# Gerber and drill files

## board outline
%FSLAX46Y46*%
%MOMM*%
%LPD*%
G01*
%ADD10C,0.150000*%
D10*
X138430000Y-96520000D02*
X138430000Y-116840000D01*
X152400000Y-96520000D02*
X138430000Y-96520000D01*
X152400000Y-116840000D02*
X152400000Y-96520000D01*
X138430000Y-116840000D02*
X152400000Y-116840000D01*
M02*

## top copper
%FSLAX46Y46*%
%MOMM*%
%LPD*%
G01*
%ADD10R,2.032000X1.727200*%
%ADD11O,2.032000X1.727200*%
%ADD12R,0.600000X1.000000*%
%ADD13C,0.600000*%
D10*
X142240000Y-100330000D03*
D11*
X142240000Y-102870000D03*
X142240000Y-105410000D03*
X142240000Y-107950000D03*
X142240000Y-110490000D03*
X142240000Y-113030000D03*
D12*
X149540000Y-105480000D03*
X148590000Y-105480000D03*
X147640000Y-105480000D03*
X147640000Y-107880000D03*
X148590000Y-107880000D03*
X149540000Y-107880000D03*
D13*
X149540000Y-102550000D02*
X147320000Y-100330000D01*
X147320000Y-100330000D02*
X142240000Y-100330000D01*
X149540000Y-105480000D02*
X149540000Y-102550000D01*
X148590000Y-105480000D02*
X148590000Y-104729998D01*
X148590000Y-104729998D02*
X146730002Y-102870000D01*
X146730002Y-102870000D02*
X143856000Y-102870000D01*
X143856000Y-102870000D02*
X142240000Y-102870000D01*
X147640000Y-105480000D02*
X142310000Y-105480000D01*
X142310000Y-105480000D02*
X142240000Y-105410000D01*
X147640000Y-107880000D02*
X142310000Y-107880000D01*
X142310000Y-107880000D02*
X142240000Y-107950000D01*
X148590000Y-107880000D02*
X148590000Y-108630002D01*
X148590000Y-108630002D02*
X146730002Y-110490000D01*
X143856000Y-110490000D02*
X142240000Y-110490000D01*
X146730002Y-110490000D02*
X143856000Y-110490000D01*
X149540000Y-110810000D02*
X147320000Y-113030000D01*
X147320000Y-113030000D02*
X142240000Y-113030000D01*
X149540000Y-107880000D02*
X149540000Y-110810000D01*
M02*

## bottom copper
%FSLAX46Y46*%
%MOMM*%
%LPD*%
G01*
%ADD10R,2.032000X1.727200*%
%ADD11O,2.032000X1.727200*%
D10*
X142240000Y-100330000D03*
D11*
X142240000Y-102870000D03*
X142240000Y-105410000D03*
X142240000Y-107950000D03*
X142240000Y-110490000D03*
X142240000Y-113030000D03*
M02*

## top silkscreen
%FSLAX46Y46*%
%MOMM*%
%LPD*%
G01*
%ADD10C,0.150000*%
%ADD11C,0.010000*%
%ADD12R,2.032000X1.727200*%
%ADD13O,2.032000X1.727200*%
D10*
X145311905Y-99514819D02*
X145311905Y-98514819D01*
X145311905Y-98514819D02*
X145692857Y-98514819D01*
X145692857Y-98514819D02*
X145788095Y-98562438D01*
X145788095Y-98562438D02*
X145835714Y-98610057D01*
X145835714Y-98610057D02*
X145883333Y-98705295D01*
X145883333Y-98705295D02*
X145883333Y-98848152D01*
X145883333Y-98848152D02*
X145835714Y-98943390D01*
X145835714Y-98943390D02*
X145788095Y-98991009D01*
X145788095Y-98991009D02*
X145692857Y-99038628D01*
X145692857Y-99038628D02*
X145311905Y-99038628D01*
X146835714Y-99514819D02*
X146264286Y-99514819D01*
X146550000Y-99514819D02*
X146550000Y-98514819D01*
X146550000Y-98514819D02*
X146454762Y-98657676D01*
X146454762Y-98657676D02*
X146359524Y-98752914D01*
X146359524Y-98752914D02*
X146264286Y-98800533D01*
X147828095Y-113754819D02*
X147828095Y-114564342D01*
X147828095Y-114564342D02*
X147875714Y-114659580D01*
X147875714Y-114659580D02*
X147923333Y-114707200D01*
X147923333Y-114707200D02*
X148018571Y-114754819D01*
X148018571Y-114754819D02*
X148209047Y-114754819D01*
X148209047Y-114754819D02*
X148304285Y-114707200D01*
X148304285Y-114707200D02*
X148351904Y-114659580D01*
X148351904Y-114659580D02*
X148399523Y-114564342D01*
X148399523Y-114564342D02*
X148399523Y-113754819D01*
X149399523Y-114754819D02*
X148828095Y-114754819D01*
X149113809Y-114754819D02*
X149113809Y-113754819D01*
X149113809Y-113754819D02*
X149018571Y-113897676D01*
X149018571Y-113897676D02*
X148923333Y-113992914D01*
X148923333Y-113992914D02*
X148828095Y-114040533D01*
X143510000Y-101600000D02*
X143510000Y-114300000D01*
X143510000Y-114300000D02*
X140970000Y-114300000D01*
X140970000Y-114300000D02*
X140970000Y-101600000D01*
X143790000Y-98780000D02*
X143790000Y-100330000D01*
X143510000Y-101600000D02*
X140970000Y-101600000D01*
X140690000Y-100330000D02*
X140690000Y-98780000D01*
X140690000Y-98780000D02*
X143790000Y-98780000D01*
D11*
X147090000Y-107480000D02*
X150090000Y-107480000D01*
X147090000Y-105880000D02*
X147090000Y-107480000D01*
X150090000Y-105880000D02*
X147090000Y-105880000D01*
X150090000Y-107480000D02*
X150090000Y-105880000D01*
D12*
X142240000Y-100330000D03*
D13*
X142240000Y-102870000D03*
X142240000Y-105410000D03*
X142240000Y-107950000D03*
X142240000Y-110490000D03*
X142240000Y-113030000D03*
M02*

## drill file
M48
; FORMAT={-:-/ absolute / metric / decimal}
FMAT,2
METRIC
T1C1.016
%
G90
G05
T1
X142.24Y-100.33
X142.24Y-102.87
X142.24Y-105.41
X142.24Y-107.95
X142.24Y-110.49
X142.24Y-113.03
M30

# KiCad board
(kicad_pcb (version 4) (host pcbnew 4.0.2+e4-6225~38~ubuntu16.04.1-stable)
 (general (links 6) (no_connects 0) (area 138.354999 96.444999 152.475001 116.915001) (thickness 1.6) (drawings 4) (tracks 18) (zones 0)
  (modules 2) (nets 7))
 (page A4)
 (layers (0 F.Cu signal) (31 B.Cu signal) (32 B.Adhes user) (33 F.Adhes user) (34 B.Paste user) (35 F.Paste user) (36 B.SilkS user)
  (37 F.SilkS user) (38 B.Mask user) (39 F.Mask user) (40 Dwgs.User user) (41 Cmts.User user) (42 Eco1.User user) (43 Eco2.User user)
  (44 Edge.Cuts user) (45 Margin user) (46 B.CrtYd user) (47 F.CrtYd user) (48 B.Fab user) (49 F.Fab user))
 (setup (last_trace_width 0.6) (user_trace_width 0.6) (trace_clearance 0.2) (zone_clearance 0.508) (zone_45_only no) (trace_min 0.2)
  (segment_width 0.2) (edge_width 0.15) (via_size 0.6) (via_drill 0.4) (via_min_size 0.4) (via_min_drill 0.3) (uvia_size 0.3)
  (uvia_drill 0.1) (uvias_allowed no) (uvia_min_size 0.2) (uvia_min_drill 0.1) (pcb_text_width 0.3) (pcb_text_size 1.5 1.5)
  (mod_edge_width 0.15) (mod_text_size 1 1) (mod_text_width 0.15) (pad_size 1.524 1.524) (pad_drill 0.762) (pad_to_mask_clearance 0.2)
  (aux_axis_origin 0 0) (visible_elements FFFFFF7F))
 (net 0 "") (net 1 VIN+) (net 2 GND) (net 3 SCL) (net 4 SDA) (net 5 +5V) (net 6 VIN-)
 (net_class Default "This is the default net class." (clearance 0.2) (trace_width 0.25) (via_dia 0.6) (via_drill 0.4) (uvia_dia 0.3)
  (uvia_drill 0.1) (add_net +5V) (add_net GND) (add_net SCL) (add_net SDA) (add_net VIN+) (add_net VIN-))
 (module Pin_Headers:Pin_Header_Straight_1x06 (layer F.Cu) (at 142.24 100.33)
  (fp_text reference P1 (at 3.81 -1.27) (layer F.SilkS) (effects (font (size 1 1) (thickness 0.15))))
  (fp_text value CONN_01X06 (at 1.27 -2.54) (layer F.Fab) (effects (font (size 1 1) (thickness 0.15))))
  (fp_line (start 1.27 1.27) (end 1.27 13.97) (layer F.SilkS) (width 0.15))
  (fp_line (start 1.27 13.97) (end -1.27 13.97) (layer F.SilkS) (width 0.15))
  (fp_line (start -1.27 13.97) (end -1.27 1.27) (layer F.SilkS) (width 0.15))
  (fp_line (start 1.55 -1.55) (end 1.55 0) (layer F.SilkS) (width 0.15))
  (fp_line (start 1.27 1.27) (end -1.27 1.27) (layer F.SilkS) (width 0.15))
  (fp_line (start -1.55 0) (end -1.55 -1.55) (layer F.SilkS) (width 0.15))
  (fp_line (start -1.55 -1.55) (end 1.55 -1.55) (layer F.SilkS) (width 0.15))
  (pad 1 thru_hole rect (at 0 0) (size 2.032 1.7272) (drill 1.016) (layers *.Cu *.Mask F.SilkS) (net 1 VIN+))
  (pad 2 thru_hole oval (at 0 2.54) (size 2.032 1.7272) (drill 1.016) (layers *.Cu *.Mask F.SilkS) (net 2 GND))
  (pad 3 thru_hole oval (at 0 5.08) (size 2.032 1.7272) (drill 1.016) (layers *.Cu *.Mask F.SilkS) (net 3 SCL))
  (pad 4 thru_hole oval (at 0 7.62) (size 2.032 1.7272) (drill 1.016) (layers *.Cu *.Mask F.SilkS) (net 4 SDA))
  (pad 5 thru_hole oval (at 0 10.16) (size 2.032 1.7272) (drill 1.016) (layers *.Cu *.Mask F.SilkS) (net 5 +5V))
  (pad 6 thru_hole oval (at 0 12.7) (size 2.032 1.7272) (drill 1.016) (layers *.Cu *.Mask F.SilkS) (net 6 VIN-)))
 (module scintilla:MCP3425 (layer F.Cu) (at 148.59 106.68 180)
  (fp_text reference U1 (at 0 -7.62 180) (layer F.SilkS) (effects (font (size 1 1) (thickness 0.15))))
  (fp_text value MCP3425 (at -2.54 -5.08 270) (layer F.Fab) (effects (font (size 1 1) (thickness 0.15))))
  (fp_line (start 1.5 -0.8) (end -1.5 -0.8) (layer F.SilkS) (width 0.01))
  (fp_line (start 1.5 0.8) (end 1.5 -0.8) (layer F.SilkS) (width 0.01))
  (fp_line (start -1.5 0.8) (end 1.5 0.8) (layer F.SilkS) (width 0.01))
  (fp_line (start -1.5 -0.8) (end -1.5 0.8) (layer F.SilkS) (width 0.01))
  (pad 1 smd rect (at -0.95 1.2 180) (size 0.6 1) (layers F.Cu F.Paste F.Mask) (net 1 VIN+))
  (pad 2 smd rect (at 0 1.2 180) (size 0.6 1) (layers F.Cu F.Paste F.Mask) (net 2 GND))
  (pad 3 smd rect (at 0.95 1.2 180) (size 0.6 1) (layers F.Cu F.Paste F.Mask) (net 3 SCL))
  (pad 4 smd rect (at 0.95 -1.2 180) (size 0.6 1) (layers F.Cu F.Paste F.Mask) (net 4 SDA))
  (pad 5 smd rect (at 0 -1.2 180) (size 0.6 1) (layers F.Cu F.Paste F.Mask) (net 5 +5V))
  (pad 6 smd rect (at -0.95 -1.2 180) (size 0.6 1) (layers F.Cu F.Paste F.Mask) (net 6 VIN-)))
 (gr_line (start 138.43 96.52) (end 138.43 116.84) (layer Edge.Cuts) (width 0.15))
 (gr_line (start 152.4 96.52) (end 138.43 96.52) (layer Edge.Cuts) (width 0.15))
 (gr_line (start 152.4 116.84) (end 152.4 96.52) (layer Edge.Cuts) (width 0.15))
 (gr_line (start 138.43 116.84) (end 152.4 116.84) (layer Edge.Cuts) (width 0.15))
 (segment (start 149.54 102.55) (end 147.32 100.33) (width 0.6) (layer F.Cu) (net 1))
 (segment (start 147.32 100.33) (end 142.24 100.33) (width 0.6) (layer F.Cu) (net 1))
 (segment (start 149.54 105.48) (end 149.54 102.55) (width 0.6) (layer F.Cu) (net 1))
 (segment (start 148.59 105.48) (end 148.59 104.729998) (width 0.6) (layer F.Cu) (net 2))
 (segment (start 148.59 104.729998) (end 146.730002 102.87) (width 0.6) (layer F.Cu) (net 2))
 (segment (start 146.730002 102.87) (end 143.856 102.87) (width 0.6) (layer F.Cu) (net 2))
 (segment (start 143.856 102.87) (end 142.24 102.87) (width 0.6) (layer F.Cu) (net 2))
 (segment (start 147.64 105.48) (end 142.31 105.48) (width 0.6) (layer F.Cu) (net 3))
 (segment (start 142.31 105.48) (end 142.24 105.41) (width 0.6) (layer F.Cu) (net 3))
 (segment (start 147.64 107.88) (end 142.31 107.88) (width 0.6) (layer F.Cu) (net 4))
 (segment (start 142.31 107.88) (end 142.24 107.95) (width 0.6) (layer F.Cu) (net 4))
 (segment (start 148.59 107.88) (end 148.59 108.630002) (width 0.6) (layer F.Cu) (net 5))
 (segment (start 148.59 108.630002) (end 146.730002 110.49) (width 0.6) (layer F.Cu) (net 5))
 (segment (start 143.856 110.49) (end 142.24 110.49) (width 0.6) (layer F.Cu) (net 5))
 (segment (start 146.730002 110.49) (end 143.856 110.49) (width 0.6) (layer F.Cu) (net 5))
 (segment (start 149.54 110.81) (end 147.32 113.03) (width 0.6) (layer F.Cu) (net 6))
 (segment (start 147.32 113.03) (end 142.24 113.03) (width 0.6) (layer F.Cu) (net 6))
 (segment (start 149.54 107.88) (end 149.54 110.81) (width 0.6) (layer F.Cu) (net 6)))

